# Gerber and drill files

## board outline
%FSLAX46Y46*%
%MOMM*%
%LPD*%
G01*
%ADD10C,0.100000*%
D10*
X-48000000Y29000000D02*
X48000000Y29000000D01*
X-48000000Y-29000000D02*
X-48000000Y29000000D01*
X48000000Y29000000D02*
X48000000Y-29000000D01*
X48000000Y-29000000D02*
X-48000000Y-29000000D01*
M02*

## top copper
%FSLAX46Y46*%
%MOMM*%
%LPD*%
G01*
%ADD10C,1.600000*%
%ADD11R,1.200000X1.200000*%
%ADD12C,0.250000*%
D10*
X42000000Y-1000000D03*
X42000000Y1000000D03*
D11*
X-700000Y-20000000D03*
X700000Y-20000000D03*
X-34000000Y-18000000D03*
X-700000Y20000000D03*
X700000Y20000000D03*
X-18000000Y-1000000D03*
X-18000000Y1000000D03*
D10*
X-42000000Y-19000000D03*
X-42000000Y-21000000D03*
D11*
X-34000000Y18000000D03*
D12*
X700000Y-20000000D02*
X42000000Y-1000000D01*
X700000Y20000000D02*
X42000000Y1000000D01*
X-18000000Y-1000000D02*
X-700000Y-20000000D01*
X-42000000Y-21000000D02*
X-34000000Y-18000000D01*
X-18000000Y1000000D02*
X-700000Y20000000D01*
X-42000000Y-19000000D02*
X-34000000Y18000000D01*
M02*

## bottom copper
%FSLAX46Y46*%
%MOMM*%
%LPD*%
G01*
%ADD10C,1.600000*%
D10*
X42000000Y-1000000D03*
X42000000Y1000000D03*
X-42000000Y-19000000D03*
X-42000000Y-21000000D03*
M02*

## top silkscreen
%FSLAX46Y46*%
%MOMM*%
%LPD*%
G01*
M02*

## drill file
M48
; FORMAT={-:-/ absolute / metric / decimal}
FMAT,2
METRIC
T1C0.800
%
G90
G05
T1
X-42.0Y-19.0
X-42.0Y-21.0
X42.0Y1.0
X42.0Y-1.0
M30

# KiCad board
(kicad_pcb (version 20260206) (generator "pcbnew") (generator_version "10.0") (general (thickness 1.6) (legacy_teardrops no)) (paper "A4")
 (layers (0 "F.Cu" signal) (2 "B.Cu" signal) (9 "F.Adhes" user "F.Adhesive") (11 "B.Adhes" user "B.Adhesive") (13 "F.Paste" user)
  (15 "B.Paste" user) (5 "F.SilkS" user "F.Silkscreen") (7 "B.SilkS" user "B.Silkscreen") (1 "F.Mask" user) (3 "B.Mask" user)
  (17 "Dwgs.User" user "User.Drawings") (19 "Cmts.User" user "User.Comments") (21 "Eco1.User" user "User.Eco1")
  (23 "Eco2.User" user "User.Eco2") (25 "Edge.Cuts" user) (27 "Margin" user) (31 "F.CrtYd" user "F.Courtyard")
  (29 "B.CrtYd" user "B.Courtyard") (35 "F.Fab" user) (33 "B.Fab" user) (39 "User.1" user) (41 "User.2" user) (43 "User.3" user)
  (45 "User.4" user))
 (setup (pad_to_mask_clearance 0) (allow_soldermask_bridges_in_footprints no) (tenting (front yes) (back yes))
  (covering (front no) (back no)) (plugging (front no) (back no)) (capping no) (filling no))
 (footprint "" (layer "F.Cu") (at 42 0)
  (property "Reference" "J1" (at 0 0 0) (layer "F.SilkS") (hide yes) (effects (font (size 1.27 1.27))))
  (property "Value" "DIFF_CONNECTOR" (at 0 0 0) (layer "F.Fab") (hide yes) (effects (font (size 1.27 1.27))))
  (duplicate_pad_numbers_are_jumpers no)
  (pad "1" thru_hole circle (at 0 1) (size 1.6 1.6) (drill 0.8) (layers "*.Cu" "*.Mask") (remove_unused_layers no) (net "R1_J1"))
  (pad "2" thru_hole circle (at 0 -1) (size 1.6 1.6) (drill 0.8) (layers "*.Cu" "*.Mask") (remove_unused_layers no) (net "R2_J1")))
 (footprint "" (layer "F.Cu") (at 0 20)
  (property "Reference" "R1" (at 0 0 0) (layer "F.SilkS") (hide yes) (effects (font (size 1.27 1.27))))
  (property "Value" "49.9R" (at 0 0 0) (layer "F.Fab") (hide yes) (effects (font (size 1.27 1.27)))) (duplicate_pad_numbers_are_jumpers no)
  (pad "1" smd rect (at -0.7 0) (size 1.2 1.2) (layers "F.Cu" "F.Mask" "F.Paste") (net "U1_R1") (thermal_bridge_angle 45))
  (pad "2" smd rect (at 0.7 0) (size 1.2 1.2) (layers "F.Cu" "F.Mask" "F.Paste") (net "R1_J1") (thermal_bridge_angle 45)))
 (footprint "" (layer "F.Cu") (at -34 18)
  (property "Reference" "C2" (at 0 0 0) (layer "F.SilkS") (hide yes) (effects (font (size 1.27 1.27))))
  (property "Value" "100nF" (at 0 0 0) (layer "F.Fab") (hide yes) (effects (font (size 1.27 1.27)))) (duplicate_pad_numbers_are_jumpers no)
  (pad "1" smd rect (at 0 0) (size 1.2 1.2) (layers "F.Cu" "F.Mask" "F.Paste") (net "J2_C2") (thermal_bridge_angle 45)))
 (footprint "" (layer "F.Cu") (at 0 -20)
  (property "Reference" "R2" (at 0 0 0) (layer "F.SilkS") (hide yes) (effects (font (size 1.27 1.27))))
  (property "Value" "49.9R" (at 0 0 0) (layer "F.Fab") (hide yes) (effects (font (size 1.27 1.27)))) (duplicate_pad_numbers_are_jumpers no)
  (pad "1" smd rect (at -0.7 0) (size 1.2 1.2) (layers "F.Cu" "F.Mask" "F.Paste") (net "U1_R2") (thermal_bridge_angle 45))
  (pad "2" smd rect (at 0.7 0) (size 1.2 1.2) (layers "F.Cu" "F.Mask" "F.Paste") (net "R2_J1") (thermal_bridge_angle 45)))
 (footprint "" (layer "F.Cu") (at -18 0)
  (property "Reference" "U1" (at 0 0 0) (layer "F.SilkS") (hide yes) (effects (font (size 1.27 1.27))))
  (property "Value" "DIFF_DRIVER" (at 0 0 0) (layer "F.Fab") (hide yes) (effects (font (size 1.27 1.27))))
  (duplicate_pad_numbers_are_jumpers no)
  (pad "1" smd rect (at 0 1) (size 1.2 1.2) (layers "F.Cu" "F.Mask" "F.Paste") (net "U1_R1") (thermal_bridge_angle 45))
  (pad "2" smd rect (at 0 -1) (size 1.2 1.2) (layers "F.Cu" "F.Mask" "F.Paste") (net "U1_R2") (thermal_bridge_angle 45)))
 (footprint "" (layer "F.Cu") (at -42 20)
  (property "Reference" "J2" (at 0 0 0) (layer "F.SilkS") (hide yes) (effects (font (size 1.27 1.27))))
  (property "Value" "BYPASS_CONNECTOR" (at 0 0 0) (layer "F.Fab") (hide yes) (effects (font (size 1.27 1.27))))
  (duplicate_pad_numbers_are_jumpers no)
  (pad "1" thru_hole circle (at 0 -1) (size 1.6 1.6) (drill 0.8) (layers "*.Cu" "*.Mask") (remove_unused_layers no) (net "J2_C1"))
  (pad "2" thru_hole circle (at 0 1) (size 1.6 1.6) (drill 0.8) (layers "*.Cu" "*.Mask") (remove_unused_layers no) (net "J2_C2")))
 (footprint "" (layer "F.Cu") (at -34 -18)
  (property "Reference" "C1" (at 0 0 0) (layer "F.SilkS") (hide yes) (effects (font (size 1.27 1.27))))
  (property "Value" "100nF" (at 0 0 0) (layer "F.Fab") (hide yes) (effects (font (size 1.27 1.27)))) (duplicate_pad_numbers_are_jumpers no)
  (pad "1" smd rect (at 0 0) (size 1.2 1.2) (layers "F.Cu" "F.Mask" "F.Paste") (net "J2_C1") (thermal_bridge_angle 45)))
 (gr_line (start -48 -29) (end 48 -29) (stroke (width 0.1) (type default)) (layer "Edge.Cuts"))
 (gr_line (start -48 29) (end -48 -29) (stroke (width 0.1) (type default)) (layer "Edge.Cuts"))
 (gr_line (start 48 -29) (end 48 29) (stroke (width 0.1) (type default)) (layer "Edge.Cuts"))
 (gr_line (start 48 29) (end -48 29) (stroke (width 0.1) (type default)) (layer "Edge.Cuts"))
 (segment (start 0.7 20) (end 42 1) (width 0.25) (layer "F.Cu") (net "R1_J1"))
 (segment (start 0.7 -20) (end 42 -1) (width 0.25) (layer "F.Cu") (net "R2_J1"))
 (segment (start -18 1) (end -0.7 20) (width 0.25) (layer "F.Cu") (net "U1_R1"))
 (segment (start -42 21) (end -34 18) (width 0.25) (layer "F.Cu") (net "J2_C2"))
 (segment (start -18 -1) (end -0.7 -20) (width 0.25) (layer "F.Cu") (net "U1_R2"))
 (segment (start -42 19) (end -34 -18) (width 0.25) (layer "F.Cu") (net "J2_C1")))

